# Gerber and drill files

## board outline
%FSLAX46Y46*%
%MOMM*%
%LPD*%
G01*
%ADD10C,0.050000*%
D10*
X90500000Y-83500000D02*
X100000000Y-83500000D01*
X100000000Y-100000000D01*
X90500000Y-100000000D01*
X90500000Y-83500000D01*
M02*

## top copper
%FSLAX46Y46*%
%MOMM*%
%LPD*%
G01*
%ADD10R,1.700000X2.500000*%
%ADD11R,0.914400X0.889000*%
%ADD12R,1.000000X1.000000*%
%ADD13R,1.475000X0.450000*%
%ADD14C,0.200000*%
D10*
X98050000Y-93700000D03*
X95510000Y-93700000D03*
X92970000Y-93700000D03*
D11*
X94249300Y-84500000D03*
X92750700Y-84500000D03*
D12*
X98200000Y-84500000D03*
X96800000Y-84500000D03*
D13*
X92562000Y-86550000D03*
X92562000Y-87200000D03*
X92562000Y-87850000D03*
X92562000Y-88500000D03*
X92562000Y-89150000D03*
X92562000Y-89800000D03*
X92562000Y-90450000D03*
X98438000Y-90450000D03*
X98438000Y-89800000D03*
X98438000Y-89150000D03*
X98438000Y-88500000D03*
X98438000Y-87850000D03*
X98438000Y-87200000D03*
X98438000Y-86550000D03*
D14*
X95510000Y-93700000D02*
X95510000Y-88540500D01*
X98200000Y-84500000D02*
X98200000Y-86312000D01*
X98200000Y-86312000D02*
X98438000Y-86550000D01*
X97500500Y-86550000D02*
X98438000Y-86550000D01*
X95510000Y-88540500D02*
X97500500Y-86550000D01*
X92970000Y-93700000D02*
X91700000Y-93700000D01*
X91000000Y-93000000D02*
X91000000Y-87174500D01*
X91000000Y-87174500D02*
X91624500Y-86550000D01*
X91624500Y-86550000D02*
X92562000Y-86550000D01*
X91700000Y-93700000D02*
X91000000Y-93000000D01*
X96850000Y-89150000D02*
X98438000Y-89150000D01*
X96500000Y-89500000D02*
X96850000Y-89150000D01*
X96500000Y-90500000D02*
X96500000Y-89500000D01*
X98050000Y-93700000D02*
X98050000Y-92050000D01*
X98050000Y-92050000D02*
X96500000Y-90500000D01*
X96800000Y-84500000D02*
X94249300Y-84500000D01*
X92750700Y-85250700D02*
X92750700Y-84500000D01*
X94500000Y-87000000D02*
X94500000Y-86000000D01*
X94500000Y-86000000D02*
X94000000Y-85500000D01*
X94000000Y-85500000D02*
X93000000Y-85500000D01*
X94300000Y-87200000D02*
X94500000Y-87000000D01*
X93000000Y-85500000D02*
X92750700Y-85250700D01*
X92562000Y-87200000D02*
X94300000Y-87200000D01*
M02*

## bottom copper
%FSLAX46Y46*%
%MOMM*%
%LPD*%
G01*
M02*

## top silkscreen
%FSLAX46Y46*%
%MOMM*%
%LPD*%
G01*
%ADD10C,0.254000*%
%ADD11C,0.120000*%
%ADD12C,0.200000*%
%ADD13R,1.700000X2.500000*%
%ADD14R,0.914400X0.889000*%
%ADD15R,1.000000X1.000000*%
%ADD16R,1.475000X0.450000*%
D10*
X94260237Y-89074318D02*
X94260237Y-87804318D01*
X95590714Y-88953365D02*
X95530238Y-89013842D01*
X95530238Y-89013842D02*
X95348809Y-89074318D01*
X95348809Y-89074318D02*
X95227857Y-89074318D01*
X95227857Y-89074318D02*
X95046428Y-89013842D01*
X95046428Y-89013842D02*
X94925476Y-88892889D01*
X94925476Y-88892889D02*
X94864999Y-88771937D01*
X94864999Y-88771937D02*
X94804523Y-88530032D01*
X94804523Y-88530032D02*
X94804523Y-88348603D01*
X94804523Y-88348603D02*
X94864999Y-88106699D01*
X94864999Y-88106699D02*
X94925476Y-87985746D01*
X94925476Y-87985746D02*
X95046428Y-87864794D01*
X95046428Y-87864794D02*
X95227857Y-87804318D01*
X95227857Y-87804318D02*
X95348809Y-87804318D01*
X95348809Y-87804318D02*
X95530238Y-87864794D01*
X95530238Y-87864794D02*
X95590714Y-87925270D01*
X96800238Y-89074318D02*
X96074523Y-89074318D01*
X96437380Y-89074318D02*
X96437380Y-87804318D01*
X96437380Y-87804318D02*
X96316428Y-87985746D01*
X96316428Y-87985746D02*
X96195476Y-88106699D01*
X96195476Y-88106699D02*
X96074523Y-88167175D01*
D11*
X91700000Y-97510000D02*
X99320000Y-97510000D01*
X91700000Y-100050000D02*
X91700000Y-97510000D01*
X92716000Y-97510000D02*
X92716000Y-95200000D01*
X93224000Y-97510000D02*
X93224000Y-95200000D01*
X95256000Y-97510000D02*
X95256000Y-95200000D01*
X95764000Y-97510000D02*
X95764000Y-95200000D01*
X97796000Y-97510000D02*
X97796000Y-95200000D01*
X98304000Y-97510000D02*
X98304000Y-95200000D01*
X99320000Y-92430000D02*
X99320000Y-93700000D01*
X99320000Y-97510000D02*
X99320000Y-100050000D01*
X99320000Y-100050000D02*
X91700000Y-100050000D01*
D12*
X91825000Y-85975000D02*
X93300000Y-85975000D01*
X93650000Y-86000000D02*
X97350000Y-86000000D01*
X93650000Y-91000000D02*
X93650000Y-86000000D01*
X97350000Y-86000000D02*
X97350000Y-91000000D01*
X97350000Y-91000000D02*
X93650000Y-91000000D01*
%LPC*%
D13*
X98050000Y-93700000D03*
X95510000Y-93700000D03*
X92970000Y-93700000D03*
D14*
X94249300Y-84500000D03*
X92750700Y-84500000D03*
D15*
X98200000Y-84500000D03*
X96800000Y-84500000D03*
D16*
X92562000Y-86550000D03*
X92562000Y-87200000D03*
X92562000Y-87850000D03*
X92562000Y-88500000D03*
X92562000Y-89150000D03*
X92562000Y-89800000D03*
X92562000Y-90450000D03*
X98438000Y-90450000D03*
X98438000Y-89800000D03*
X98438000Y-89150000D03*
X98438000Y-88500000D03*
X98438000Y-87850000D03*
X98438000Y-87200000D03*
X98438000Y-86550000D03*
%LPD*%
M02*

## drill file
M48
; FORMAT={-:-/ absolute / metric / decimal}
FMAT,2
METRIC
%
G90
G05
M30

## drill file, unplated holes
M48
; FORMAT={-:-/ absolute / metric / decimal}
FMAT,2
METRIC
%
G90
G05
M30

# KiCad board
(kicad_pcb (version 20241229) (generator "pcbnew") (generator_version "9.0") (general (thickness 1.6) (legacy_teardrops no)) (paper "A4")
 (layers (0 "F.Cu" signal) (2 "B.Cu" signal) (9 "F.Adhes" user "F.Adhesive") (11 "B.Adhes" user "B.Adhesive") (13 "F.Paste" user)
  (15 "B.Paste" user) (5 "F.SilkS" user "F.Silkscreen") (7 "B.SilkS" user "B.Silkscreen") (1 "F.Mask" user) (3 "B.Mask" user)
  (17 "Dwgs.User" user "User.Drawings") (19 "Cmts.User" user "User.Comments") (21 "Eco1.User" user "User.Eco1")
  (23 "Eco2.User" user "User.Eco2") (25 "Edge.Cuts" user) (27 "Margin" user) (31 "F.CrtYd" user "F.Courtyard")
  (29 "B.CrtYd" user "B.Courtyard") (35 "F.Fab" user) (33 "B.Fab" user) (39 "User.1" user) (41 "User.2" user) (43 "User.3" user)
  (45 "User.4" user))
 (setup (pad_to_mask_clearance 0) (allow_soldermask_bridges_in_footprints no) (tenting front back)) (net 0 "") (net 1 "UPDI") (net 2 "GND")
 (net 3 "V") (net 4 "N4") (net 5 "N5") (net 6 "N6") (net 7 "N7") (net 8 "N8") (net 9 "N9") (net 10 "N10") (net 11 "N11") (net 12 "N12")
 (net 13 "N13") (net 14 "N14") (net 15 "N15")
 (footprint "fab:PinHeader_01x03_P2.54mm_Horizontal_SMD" (layer "F.Cu") (at 98.05 93.7 -90)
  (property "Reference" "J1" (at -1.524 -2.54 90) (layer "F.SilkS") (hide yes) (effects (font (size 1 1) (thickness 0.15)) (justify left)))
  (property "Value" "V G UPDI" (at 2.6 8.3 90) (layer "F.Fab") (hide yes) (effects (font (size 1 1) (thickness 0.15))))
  (fp_line (start 3.81 6.35) (end 3.81 -1.27) (stroke (width 0.12) (type solid)) (layer "F.SilkS"))
  (fp_line (start 6.35 6.35) (end 3.81 6.35) (stroke (width 0.12) (type solid)) (layer "F.SilkS"))
  (fp_line (start 3.81 5.334) (end 1.5 5.334) (stroke (width 0.12) (type solid)) (layer "F.SilkS"))
  (fp_line (start 3.81 4.826) (end 1.5 4.826) (stroke (width 0.12) (type solid)) (layer "F.SilkS"))
  (fp_line (start 3.81 2.794) (end 1.5 2.794) (stroke (width 0.12) (type solid)) (layer "F.SilkS"))
  (fp_line (start 3.81 2.286) (end 1.5 2.286) (stroke (width 0.12) (type solid)) (layer "F.SilkS"))
  (fp_line (start 3.81 0.254) (end 1.5 0.254) (stroke (width 0.12) (type solid)) (layer "F.SilkS"))
  (fp_line (start 3.81 -0.254) (end 1.5 -0.254) (stroke (width 0.12) (type solid)) (layer "F.SilkS"))
  (fp_line (start -1.27 -1.27) (end 0 -1.27) (stroke (width 0.12) (type solid)) (layer "F.SilkS"))
  (fp_line (start 3.81 -1.27) (end 6.35 -1.27) (stroke (width 0.12) (type solid)) (layer "F.SilkS"))
  (fp_line (start 6.35 -1.27) (end 6.35 6.35) (stroke (width 0.12) (type solid)) (layer "F.SilkS"))
  (pad "1" smd rect (at 0 0 270) (size 2.5 1.7) (layers "F.Cu" "F.Mask" "F.Paste") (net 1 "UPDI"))
  (pad "2" smd rect (at 0 2.54 270) (size 2.5 1.7) (layers "F.Cu" "F.Mask" "F.Paste") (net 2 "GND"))
  (pad "3" smd rect (at 0 5.08 270) (size 2.5 1.7) (layers "F.Cu" "F.Mask" "F.Paste") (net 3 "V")))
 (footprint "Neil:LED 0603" (layer "F.Cu") (at 93.5 84.5 180)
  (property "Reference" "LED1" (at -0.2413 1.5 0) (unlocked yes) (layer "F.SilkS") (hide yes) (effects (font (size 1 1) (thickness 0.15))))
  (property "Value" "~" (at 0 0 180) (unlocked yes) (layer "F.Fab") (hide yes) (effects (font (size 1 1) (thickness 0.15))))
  (pad "1" smd rect (at -0.7493 0 180) (size 0.9144 0.889) (layers "F.Cu" "F.Mask" "F.Paste") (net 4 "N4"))
  (pad "2" smd rect (at 0.7493 0 180) (size 0.9144 0.889) (layers "F.Cu" "F.Mask" "F.Paste") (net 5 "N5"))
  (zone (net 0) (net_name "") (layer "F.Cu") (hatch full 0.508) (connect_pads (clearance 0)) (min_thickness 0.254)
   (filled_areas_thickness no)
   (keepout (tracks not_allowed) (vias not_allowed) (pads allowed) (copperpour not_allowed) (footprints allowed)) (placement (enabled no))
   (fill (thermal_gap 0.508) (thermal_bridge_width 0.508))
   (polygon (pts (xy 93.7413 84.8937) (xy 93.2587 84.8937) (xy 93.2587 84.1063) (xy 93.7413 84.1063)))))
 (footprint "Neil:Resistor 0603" (layer "F.Cu") (at 97.5 84.5 180)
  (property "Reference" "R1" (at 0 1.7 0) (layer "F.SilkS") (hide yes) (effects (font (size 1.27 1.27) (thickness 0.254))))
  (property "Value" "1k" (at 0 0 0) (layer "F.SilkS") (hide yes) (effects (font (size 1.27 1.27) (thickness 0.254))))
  (pad "1" smd rect (at -0.7 0 270) (size 1 1) (layers "F.Cu" "F.Mask" "F.Paste") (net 2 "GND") (thermal_bridge_angle 45))
  (pad "2" smd rect (at 0.7 0 270) (size 1 1) (layers "F.Cu" "F.Mask" "F.Paste") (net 4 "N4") (thermal_bridge_angle 45)))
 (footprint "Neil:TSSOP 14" (layer "F.Cu") (at 95.5 88.5)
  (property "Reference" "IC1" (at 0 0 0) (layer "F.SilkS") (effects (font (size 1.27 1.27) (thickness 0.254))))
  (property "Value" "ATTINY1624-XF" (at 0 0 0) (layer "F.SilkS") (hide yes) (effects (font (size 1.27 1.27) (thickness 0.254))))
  (fp_line (start -3.675 -2.525) (end -2.2 -2.525) (stroke (width 0.2) (type solid)) (layer "F.SilkS"))
  (fp_line (start -1.85 -2.5) (end 1.85 -2.5) (stroke (width 0.2) (type solid)) (layer "F.SilkS"))
  (fp_line (start -1.85 2.5) (end -1.85 -2.5) (stroke (width 0.2) (type solid)) (layer "F.SilkS"))
  (fp_line (start 1.85 -2.5) (end 1.85 2.5) (stroke (width 0.2) (type solid)) (layer "F.SilkS"))
  (fp_line (start 1.85 2.5) (end -1.85 2.5) (stroke (width 0.2) (type solid)) (layer "F.SilkS"))
  (pad "1" smd rect (at -2.938 -1.95 90) (size 0.45 1.475) (layers "F.Cu" "F.Mask" "F.Paste") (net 3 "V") (thermal_bridge_angle 45))
  (pad "2" smd rect (at -2.938 -1.3 90) (size 0.45 1.475) (layers "F.Cu" "F.Mask" "F.Paste") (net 5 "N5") (thermal_bridge_angle 45))
  (pad "3" smd rect (at -2.938 -0.65 90) (size 0.45 1.475) (layers "F.Cu" "F.Mask" "F.Paste") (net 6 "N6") (thermal_bridge_angle 45))
  (pad "4" smd rect (at -2.938 0 90) (size 0.45 1.475) (layers "F.Cu" "F.Mask" "F.Paste") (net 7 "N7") (thermal_bridge_angle 45))
  (pad "5" smd rect (at -2.938 0.65 90) (size 0.45 1.475) (layers "F.Cu" "F.Mask" "F.Paste") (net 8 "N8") (thermal_bridge_angle 45))
  (pad "6" smd rect (at -2.938 1.3 90) (size 0.45 1.475) (layers "F.Cu" "F.Mask" "F.Paste") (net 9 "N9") (thermal_bridge_angle 45))
  (pad "7" smd rect (at -2.938 1.95 90) (size 0.45 1.475) (layers "F.Cu" "F.Mask" "F.Paste") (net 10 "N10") (thermal_bridge_angle 45))
  (pad "8" smd rect (at 2.938 1.95 90) (size 0.45 1.475) (layers "F.Cu" "F.Mask" "F.Paste") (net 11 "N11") (thermal_bridge_angle 45))
  (pad "9" smd rect (at 2.938 1.3 90) (size 0.45 1.475) (layers "F.Cu" "F.Mask" "F.Paste") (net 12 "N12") (thermal_bridge_angle 45))
  (pad "10" smd rect (at 2.938 0.65 90) (size 0.45 1.475) (layers "F.Cu" "F.Mask" "F.Paste") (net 1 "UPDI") (thermal_bridge_angle 45))
  (pad "11" smd rect (at 2.938 0 90) (size 0.45 1.475) (layers "F.Cu" "F.Mask" "F.Paste") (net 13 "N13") (thermal_bridge_angle 45))
  (pad "12" smd rect (at 2.938 -0.65 90) (size 0.45 1.475) (layers "F.Cu" "F.Mask" "F.Paste") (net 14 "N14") (thermal_bridge_angle 45))
  (pad "13" smd rect (at 2.938 -1.3 90) (size 0.45 1.475) (layers "F.Cu" "F.Mask" "F.Paste") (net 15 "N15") (thermal_bridge_angle 45))
  (pad "14" smd rect (at 2.938 -1.95 90) (size 0.45 1.475) (layers "F.Cu" "F.Mask" "F.Paste") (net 2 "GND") (thermal_bridge_angle 45)))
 (gr_rect (start 90.5 83.5) (end 100 100) (stroke (width 0.05) (type default)) (fill no) (layer "Edge.Cuts"))
 (segment (start 95.51 93.7) (end 95.51 88.5405) (width 0.2) (layer "F.Cu") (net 2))
 (segment (start 98.2 84.5) (end 98.2 86.312) (width 0.2) (layer "F.Cu") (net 2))
 (segment (start 98.2 86.312) (end 98.438 86.55) (width 0.2) (layer "F.Cu") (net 2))
 (segment (start 97.5005 86.55) (end 98.438 86.55) (width 0.2) (layer "F.Cu") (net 2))
 (segment (start 95.51 88.5405) (end 97.5005 86.55) (width 0.2) (layer "F.Cu") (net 2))
 (segment (start 92.97 93.7) (end 91.7 93.7) (width 0.2) (layer "F.Cu") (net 3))
 (segment (start 91 93) (end 91 87.1745) (width 0.2) (layer "F.Cu") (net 3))
 (segment (start 91 87.1745) (end 91.6245 86.55) (width 0.2) (layer "F.Cu") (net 3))
 (segment (start 91.6245 86.55) (end 92.562 86.55) (width 0.2) (layer "F.Cu") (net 3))
 (segment (start 91.7 93.7) (end 91 93) (width 0.2) (layer "F.Cu") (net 3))
 (segment (start 96.85 89.15) (end 98.438 89.15) (width 0.2) (layer "F.Cu") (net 1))
 (segment (start 96.5 89.5) (end 96.85 89.15) (width 0.2) (layer "F.Cu") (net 1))
 (segment (start 96.5 90.5) (end 96.5 89.5) (width 0.2) (layer "F.Cu") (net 1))
 (segment (start 98.05 93.7) (end 98.05 92.05) (width 0.2) (layer "F.Cu") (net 1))
 (segment (start 98.05 92.05) (end 96.5 90.5) (width 0.2) (layer "F.Cu") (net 1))
 (segment (start 96.8 84.5) (end 94.2493 84.5) (width 0.2) (layer "F.Cu") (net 4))
 (segment (start 92.7507 85.2507) (end 92.7507 84.5) (width 0.2) (layer "F.Cu") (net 5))
 (segment (start 94.5 87) (end 94.5 86) (width 0.2) (layer "F.Cu") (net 5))
 (segment (start 94.5 86) (end 94 85.5) (width 0.2) (layer "F.Cu") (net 5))
 (segment (start 94 85.5) (end 93 85.5) (width 0.2) (layer "F.Cu") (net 5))
 (segment (start 94.3 87.2) (end 94.5 87) (width 0.2) (layer "F.Cu") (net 5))
 (segment (start 93 85.5) (end 92.7507 85.2507) (width 0.2) (layer "F.Cu") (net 5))
 (segment (start 92.562 87.2) (end 94.3 87.2) (width 0.2) (layer "F.Cu") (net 5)))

